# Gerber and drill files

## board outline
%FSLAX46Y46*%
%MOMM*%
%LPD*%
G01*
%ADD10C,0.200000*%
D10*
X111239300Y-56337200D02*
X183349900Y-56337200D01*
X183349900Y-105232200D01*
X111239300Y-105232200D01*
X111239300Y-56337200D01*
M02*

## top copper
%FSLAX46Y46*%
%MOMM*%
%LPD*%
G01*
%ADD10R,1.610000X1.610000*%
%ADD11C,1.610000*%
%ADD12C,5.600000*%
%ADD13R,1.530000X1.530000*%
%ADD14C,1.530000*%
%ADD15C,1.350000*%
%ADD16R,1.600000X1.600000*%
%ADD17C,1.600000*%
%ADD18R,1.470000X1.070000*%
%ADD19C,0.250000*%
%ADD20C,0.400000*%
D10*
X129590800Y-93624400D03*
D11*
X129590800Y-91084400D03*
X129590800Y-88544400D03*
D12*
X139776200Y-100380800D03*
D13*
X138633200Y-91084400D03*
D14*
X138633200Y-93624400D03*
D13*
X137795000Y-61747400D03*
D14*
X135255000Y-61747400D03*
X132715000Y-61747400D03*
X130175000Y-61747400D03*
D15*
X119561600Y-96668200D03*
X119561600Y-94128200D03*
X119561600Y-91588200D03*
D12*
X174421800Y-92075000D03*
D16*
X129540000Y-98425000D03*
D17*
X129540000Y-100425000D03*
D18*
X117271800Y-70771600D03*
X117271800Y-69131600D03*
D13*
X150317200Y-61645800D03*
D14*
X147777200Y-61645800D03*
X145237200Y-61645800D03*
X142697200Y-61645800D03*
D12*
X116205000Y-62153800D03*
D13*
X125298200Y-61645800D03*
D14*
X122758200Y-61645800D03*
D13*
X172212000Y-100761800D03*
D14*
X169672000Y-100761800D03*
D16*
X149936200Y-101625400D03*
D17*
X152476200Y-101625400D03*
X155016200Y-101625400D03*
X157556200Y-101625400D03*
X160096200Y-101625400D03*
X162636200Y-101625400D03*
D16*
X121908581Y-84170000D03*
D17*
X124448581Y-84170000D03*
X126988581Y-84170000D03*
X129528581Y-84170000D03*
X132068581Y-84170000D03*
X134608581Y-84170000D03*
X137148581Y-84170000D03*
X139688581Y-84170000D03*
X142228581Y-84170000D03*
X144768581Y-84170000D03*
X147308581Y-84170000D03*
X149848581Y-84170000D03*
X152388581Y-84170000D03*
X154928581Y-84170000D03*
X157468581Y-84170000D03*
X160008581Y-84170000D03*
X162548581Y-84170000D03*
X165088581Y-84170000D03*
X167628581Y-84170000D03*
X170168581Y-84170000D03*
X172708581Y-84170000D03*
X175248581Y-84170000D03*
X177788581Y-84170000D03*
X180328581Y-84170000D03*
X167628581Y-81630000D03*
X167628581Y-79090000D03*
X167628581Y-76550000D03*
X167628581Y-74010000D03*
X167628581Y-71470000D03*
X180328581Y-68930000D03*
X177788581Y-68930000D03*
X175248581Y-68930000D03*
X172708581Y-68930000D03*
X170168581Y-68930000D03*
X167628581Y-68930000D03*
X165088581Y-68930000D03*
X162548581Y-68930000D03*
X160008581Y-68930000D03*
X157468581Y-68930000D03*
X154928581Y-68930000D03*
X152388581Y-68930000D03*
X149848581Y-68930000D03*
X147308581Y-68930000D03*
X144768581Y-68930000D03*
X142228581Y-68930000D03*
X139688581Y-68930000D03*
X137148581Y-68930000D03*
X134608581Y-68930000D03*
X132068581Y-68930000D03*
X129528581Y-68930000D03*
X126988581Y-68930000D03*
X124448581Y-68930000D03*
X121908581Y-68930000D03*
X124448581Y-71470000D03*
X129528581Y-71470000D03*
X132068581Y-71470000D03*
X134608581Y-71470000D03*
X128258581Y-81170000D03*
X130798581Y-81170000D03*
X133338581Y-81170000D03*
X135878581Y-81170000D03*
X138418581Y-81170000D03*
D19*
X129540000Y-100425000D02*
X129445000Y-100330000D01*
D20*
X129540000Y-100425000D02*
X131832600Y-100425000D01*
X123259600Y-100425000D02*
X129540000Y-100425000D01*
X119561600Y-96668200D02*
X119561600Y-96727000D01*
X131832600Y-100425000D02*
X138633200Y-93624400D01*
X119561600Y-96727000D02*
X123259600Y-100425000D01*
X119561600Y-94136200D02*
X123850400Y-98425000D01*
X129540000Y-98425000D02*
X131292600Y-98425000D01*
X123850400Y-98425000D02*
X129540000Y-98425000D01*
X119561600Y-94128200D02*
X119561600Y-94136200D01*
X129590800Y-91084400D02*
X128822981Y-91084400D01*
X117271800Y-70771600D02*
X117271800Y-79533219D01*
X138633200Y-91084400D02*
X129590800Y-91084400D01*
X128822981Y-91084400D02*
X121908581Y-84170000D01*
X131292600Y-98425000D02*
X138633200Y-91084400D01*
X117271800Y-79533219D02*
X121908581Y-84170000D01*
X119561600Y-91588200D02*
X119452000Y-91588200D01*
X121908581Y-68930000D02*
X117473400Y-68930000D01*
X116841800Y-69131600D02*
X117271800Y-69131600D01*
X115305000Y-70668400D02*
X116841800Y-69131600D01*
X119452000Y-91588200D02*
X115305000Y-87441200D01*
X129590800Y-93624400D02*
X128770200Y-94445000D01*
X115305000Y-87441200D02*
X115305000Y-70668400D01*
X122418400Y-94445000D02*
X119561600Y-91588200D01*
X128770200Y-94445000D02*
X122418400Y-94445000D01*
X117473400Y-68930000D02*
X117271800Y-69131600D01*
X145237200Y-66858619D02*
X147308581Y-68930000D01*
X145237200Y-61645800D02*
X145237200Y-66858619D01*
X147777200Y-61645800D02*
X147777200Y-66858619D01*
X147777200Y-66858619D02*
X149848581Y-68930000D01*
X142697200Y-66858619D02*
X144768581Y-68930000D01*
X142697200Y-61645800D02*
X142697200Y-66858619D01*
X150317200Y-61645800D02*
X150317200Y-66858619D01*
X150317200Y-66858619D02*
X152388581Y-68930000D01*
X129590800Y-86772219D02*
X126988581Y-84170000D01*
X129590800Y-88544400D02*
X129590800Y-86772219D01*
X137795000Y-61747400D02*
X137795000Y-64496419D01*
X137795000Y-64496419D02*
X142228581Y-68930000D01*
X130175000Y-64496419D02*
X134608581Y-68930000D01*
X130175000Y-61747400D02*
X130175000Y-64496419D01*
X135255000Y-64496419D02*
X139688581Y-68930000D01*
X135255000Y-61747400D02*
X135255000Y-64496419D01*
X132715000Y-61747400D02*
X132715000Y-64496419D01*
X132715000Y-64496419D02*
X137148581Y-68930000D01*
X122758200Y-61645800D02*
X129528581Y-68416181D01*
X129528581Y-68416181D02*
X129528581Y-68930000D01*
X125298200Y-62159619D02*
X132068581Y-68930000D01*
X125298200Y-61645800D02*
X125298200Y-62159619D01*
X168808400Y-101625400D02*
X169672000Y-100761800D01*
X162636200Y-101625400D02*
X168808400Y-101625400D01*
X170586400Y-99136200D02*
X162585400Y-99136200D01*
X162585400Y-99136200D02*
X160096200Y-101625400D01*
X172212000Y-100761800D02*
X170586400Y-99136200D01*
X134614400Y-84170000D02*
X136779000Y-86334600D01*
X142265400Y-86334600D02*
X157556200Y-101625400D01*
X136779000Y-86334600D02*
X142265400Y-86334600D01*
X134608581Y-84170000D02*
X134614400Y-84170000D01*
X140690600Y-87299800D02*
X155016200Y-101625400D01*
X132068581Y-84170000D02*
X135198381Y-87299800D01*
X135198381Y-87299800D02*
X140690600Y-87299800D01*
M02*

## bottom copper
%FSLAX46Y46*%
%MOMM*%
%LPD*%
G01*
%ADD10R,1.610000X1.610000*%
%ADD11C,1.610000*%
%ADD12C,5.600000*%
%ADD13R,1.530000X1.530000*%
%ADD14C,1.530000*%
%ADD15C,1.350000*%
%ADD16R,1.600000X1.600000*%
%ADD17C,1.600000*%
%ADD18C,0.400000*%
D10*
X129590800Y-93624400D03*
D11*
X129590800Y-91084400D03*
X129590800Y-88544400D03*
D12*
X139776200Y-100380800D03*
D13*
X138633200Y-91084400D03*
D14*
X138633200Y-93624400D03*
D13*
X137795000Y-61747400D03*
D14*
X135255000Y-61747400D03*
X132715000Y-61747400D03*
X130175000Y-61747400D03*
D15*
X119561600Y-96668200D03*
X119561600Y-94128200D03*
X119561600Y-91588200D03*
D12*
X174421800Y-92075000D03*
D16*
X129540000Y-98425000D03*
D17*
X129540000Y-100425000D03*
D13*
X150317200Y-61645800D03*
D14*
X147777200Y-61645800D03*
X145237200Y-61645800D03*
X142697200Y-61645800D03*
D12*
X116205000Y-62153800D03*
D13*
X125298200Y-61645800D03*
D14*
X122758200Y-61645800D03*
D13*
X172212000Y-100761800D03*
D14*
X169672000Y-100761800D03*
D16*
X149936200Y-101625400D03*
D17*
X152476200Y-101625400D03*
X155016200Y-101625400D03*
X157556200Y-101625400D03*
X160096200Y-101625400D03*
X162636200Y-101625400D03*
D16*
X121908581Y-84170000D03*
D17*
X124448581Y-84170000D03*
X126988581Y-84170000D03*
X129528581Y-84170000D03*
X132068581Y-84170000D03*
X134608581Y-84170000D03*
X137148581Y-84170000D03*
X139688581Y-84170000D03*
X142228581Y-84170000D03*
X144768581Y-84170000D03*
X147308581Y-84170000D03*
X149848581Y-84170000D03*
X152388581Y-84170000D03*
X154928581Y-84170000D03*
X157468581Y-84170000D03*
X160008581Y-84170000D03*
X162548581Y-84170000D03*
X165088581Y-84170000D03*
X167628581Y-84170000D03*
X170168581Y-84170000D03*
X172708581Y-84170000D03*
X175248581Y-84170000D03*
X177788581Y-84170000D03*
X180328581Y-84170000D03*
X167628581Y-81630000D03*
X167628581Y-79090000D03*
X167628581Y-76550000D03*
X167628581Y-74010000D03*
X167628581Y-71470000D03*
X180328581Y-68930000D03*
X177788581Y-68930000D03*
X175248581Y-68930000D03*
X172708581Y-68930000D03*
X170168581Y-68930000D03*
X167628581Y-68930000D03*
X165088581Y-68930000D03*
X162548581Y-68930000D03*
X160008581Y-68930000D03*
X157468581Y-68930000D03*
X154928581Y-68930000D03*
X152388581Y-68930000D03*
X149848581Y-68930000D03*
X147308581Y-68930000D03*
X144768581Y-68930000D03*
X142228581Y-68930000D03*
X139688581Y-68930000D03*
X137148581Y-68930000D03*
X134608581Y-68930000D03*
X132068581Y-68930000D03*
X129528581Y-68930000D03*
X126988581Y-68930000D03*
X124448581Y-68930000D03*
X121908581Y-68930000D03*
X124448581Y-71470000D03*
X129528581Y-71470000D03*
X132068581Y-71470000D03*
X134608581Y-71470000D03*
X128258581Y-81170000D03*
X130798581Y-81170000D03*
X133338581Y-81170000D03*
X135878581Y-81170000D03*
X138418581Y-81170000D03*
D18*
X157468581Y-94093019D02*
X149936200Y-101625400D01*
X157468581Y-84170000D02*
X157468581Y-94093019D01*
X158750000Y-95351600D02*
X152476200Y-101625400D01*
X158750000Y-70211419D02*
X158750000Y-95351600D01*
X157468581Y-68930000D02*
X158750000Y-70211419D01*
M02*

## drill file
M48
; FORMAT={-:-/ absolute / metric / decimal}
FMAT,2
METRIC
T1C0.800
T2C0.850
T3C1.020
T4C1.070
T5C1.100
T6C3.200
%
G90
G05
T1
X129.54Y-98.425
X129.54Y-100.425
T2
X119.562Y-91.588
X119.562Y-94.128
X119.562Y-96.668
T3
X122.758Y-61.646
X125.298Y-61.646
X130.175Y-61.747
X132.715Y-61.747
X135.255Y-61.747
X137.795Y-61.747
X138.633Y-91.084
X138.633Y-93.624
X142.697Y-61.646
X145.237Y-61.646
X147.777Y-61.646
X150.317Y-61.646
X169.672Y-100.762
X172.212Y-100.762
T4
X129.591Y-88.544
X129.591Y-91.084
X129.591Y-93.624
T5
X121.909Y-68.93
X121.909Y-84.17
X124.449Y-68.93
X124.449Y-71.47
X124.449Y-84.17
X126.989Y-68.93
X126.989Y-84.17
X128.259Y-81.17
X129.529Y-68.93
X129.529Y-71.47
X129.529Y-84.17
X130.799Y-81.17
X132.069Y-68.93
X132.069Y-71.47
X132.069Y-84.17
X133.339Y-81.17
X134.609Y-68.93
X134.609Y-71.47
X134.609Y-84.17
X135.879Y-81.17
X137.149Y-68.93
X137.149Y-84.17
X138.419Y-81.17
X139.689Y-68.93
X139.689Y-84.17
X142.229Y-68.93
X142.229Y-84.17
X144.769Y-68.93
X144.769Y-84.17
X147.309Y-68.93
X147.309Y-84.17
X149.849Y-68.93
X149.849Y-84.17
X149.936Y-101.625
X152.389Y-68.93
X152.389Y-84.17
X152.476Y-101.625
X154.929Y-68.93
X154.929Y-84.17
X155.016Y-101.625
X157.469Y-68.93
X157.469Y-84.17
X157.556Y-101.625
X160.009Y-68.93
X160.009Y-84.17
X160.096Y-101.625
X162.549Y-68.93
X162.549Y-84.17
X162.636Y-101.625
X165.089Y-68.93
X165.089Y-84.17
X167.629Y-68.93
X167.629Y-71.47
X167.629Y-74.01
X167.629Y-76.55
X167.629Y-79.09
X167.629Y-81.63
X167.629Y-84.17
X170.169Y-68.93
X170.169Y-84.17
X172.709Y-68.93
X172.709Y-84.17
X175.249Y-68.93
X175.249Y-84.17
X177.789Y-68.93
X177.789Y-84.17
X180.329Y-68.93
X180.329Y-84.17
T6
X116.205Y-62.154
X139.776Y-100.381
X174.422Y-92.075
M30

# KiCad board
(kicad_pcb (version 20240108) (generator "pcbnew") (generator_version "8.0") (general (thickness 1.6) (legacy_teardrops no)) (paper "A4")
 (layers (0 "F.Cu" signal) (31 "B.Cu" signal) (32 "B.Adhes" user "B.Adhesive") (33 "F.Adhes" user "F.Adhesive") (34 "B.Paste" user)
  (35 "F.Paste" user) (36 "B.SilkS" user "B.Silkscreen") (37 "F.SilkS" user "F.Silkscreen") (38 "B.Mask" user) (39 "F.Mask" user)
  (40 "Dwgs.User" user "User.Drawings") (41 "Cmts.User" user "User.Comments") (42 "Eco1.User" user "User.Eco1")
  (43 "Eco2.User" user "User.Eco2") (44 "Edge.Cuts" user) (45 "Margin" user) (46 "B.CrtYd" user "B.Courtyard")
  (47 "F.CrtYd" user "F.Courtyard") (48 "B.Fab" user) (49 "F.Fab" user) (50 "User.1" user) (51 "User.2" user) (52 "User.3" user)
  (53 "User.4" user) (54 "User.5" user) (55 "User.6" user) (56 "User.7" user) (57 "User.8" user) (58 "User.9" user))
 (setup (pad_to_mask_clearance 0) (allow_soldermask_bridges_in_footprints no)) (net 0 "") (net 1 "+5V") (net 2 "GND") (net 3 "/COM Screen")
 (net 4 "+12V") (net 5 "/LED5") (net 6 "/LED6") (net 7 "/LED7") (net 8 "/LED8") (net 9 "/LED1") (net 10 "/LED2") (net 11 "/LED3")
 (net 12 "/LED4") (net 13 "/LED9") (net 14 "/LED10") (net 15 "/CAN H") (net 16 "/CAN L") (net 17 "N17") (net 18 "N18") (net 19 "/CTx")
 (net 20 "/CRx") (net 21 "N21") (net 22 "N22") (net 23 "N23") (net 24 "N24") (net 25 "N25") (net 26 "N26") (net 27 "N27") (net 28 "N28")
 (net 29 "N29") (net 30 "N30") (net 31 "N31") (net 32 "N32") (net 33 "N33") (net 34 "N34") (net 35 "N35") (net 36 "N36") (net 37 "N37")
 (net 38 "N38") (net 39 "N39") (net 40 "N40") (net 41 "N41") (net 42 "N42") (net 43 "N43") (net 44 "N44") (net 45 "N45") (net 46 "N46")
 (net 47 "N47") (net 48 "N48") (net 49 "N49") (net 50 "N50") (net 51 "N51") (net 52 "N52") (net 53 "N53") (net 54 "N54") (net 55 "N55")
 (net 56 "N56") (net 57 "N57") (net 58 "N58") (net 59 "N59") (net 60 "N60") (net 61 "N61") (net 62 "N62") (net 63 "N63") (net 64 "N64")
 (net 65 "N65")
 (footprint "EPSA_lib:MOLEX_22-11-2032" (layer "F.Cu") (at 129.5908 93.6244 90)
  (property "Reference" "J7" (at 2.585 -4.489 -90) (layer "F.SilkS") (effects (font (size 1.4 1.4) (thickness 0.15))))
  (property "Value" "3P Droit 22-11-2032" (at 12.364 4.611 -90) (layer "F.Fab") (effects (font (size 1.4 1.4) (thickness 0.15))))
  (pad "1" thru_hole rect (at 0 0 90) (size 1.61 1.61) (drill 1.07) (layers "*.Cu" "*.Mask") (remove_unused_layers no) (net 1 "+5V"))
  (pad "2" thru_hole circle (at 2.54 0 90) (size 1.61 1.61) (drill 1.07) (layers "*.Cu" "*.Mask") (remove_unused_layers no) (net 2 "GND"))
  (pad "3" thru_hole circle (at 5.08 0 90) (size 1.61 1.61) (drill 1.07) (layers "*.Cu" "*.Mask") (remove_unused_layers no)
   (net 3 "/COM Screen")))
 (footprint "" (layer "F.Cu") (at 139.7762 100.3808)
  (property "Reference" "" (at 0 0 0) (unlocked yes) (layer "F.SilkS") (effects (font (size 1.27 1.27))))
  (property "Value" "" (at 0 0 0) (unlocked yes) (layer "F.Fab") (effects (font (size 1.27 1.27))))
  (pad "1" thru_hole circle (at 0 0) (size 5.6 5.6) (drill 3.2) (layers "*.Cu" "*.Mask") (remove_unused_layers no)))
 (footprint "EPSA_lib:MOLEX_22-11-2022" (layer "F.Cu") (at 138.6332 91.0844 -90)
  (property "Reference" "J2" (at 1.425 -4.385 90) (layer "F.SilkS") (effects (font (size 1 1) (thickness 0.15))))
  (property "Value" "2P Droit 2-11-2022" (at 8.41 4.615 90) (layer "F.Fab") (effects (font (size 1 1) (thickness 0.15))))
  (pad "1" thru_hole rect (at 0 0 270) (size 1.53 1.53) (drill 1.02) (layers "*.Cu" "*.Mask") (remove_unused_layers no) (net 2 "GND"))
  (pad "2" thru_hole circle (at 2.54 0 270) (size 1.53 1.53) (drill 1.02) (layers "*.Cu" "*.Mask") (remove_unused_layers no) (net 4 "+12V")))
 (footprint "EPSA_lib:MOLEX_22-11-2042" (layer "F.Cu") (at 133.985 61.7474 180)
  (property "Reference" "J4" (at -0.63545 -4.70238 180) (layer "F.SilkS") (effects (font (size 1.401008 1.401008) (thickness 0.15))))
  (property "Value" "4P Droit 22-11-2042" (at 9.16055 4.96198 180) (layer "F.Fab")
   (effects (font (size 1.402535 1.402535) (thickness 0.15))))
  (pad "1" thru_hole rect (at -3.81 0 180) (size 1.53 1.53) (drill 1.02) (layers "*.Cu" "*.Mask") (remove_unused_layers no) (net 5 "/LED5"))
  (pad "2" thru_hole circle (at -1.27 0 180) (size 1.53 1.53) (drill 1.02) (layers "*.Cu" "*.Mask") (remove_unused_layers no)
   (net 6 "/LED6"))
  (pad "3" thru_hole circle (at 1.27 0 180) (size 1.53 1.53) (drill 1.02) (layers "*.Cu" "*.Mask") (remove_unused_layers no) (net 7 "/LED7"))
  (pad "4" thru_hole circle (at 3.81 0 180) (size 1.53 1.53) (drill 1.02) (layers "*.Cu" "*.Mask") (remove_unused_layers no) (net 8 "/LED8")))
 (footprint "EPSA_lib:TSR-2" (layer "F.Cu") (at 115.6716 101.1682 90)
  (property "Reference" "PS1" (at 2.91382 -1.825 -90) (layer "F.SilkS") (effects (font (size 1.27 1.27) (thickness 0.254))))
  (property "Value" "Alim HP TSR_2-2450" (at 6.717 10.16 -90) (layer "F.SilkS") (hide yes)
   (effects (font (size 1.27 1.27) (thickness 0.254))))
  (pad "1" thru_hole circle (at 4.5 3.89 90) (size 1.35 1.35) (drill 0.85) (layers "*.Cu" "*.Mask") (remove_unused_layers no) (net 4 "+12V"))
  (pad "2" thru_hole circle (at 7.04 3.89 90) (size 1.35 1.35) (drill 0.85) (layers "*.Cu" "*.Mask") (remove_unused_layers no) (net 2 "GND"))
  (pad "3" thru_hole circle (at 9.58 3.89 90) (size 1.35 1.35) (drill 0.85) (layers "*.Cu" "*.Mask") (remove_unused_layers no) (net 1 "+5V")))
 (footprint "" (layer "F.Cu") (at 174.4218 92.075)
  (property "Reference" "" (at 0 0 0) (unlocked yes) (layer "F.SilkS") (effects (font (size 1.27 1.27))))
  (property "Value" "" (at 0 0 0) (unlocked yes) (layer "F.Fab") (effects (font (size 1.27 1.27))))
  (pad "1" thru_hole circle (at 0 0) (size 5.6 5.6) (drill 3.2) (layers "*.Cu" "*.Mask") (remove_unused_layers no)))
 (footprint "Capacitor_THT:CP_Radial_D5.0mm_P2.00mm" (layer "F.Cu") (at 129.54 98.425 -90)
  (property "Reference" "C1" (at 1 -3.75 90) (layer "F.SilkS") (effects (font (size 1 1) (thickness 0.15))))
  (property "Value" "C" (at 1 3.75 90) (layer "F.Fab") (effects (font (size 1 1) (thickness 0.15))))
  (pad "1" thru_hole rect (at 0 0 270) (size 1.6 1.6) (drill 0.8) (layers "*.Cu" "*.Mask") (remove_unused_layers no) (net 2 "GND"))
  (pad "2" thru_hole circle (at 2 0 270) (size 1.6 1.6) (drill 0.8) (layers "*.Cu" "*.Mask") (remove_unused_layers no) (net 4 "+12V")))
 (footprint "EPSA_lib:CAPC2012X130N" (layer "F.Cu") (at 117.2718 69.9516 90)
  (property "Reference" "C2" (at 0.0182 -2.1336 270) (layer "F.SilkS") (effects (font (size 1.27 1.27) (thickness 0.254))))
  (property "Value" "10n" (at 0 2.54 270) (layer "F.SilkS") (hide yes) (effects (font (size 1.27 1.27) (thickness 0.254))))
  (pad "1" smd rect (at -0.82 0 90) (size 1.07 1.47) (layers "F.Cu" "F.Paste" "F.Mask") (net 2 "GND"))
  (pad "2" smd rect (at 0.82 0 90) (size 1.07 1.47) (layers "F.Cu" "F.Paste" "F.Mask") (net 1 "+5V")))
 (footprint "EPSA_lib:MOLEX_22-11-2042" (layer "F.Cu") (at 146.5072 61.6458 180)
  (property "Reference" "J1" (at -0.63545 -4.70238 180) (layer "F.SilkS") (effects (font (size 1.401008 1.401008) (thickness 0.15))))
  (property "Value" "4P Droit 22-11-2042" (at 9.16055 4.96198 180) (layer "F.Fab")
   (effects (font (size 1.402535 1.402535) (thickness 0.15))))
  (pad "1" thru_hole rect (at -3.81 0 180) (size 1.53 1.53) (drill 1.02) (layers "*.Cu" "*.Mask") (remove_unused_layers no) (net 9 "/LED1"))
  (pad "2" thru_hole circle (at -1.27 0 180) (size 1.53 1.53) (drill 1.02) (layers "*.Cu" "*.Mask") (remove_unused_layers no)
   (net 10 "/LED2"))
  (pad "3" thru_hole circle (at 1.27 0 180) (size 1.53 1.53) (drill 1.02) (layers "*.Cu" "*.Mask") (remove_unused_layers no)
   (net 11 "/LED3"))
  (pad "4" thru_hole circle (at 3.81 0 180) (size 1.53 1.53) (drill 1.02) (layers "*.Cu" "*.Mask") (remove_unused_layers no)
   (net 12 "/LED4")))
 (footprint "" (layer "F.Cu") (at 116.205 62.1538)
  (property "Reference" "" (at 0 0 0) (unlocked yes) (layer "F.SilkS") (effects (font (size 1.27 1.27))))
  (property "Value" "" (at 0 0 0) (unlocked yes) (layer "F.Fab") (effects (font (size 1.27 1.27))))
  (pad "1" thru_hole circle (at 0 0) (size 5.6 5.6) (drill 3.2) (layers "*.Cu" "*.Mask") (remove_unused_layers no)))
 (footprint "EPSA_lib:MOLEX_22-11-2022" (layer "F.Cu") (at 125.2982 61.6458 180)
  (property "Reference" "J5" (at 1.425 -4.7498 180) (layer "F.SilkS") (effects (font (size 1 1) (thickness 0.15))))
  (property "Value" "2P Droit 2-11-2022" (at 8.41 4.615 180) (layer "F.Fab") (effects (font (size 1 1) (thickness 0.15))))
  (pad "1" thru_hole rect (at 0 0 180) (size 1.53 1.53) (drill 1.02) (layers "*.Cu" "*.Mask") (remove_unused_layers no) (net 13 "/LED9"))
  (pad "2" thru_hole circle (at 2.54 0 180) (size 1.53 1.53) (drill 1.02) (layers "*.Cu" "*.Mask") (remove_unused_layers no)
   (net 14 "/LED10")))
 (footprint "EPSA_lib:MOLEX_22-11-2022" (layer "F.Cu") (at 172.212 100.7618 180)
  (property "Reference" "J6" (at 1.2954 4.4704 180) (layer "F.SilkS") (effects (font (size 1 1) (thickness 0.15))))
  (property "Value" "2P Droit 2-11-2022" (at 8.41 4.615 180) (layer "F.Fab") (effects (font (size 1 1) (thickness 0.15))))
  (pad "1" thru_hole rect (at 0 0 180) (size 1.53 1.53) (drill 1.02) (layers "*.Cu" "*.Mask") (remove_unused_layers no) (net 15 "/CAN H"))
  (pad "2" thru_hole circle (at 2.54 0 180) (size 1.53 1.53) (drill 1.02) (layers "*.Cu" "*.Mask") (remove_unused_layers no)
   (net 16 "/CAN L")))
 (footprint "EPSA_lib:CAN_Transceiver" (layer "F.Cu") (at 147.3962 104.1654)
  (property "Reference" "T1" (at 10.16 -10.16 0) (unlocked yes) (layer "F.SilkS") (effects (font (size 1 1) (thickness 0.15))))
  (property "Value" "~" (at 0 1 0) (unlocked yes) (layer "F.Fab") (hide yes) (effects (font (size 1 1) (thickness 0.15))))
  (pad "1" thru_hole rect (at 2.54 -2.54) (size 1.6 1.6) (drill 1.1) (layers "*.Cu" "*.Mask") (remove_unused_layers no) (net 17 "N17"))
  (pad "2" thru_hole circle (at 5.08 -2.54) (size 1.6 1.6) (drill 1.1) (layers "*.Cu" "*.Mask") (remove_unused_layers no) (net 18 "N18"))
  (pad "3" thru_hole circle (at 7.62 -2.54) (size 1.6 1.6) (drill 1.1) (layers "*.Cu" "*.Mask") (remove_unused_layers no) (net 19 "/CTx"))
  (pad "4" thru_hole circle (at 10.16 -2.54) (size 1.6 1.6) (drill 1.1) (layers "*.Cu" "*.Mask") (remove_unused_layers no) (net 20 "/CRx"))
  (pad "5" thru_hole circle (at 12.7 -2.54) (size 1.6 1.6) (drill 1.1) (layers "*.Cu" "*.Mask") (remove_unused_layers no) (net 15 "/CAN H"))
  (pad "6" thru_hole circle (at 15.24 -2.54) (size 1.6 1.6) (drill 1.1) (layers "*.Cu" "*.Mask") (remove_unused_layers no) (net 16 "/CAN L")))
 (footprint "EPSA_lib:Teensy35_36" (layer "F.Cu") (at 151.118581 76.55)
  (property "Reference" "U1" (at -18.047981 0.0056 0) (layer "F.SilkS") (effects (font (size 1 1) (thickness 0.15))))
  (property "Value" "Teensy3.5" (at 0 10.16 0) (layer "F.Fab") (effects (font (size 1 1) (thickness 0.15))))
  (pad "1" thru_hole rect (at -29.21 7.62) (size 1.6 1.6) (drill 1.1) (layers "*.Cu" "*.Mask") (remove_unused_layers no) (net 2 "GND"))
  (pad "2" thru_hole circle (at -26.67 7.62) (size 1.6 1.6) (drill 1.1) (layers "*.Cu" "*.Mask") (remove_unused_layers no) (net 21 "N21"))
  (pad "3" thru_hole circle (at -24.13 7.62) (size 1.6 1.6) (drill 1.1) (layers "*.Cu" "*.Mask") (remove_unused_layers no)
   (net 3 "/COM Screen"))
  (pad "4" thru_hole circle (at -21.59 7.62) (size 1.6 1.6) (drill 1.1) (layers "*.Cu" "*.Mask") (remove_unused_layers no) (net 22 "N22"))
  (pad "5" thru_hole circle (at -19.05 7.62) (size 1.6 1.6) (drill 1.1) (layers "*.Cu" "*.Mask") (remove_unused_layers no) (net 19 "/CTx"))
  (pad "6" thru_hole circle (at -16.51 7.62) (size 1.6 1.6) (drill 1.1) (layers "*.Cu" "*.Mask") (remove_unused_layers no) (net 20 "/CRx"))
  (pad "7" thru_hole circle (at -13.97 7.62) (size 1.6 1.6) (drill 1.1) (layers "*.Cu" "*.Mask") (remove_unused_layers no) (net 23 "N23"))
  (pad "8" thru_hole circle (at -11.43 7.62) (size 1.6 1.6) (drill 1.1) (layers "*.Cu" "*.Mask") (remove_unused_layers no) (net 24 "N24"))
  (pad "9" thru_hole circle (at -8.89 7.62) (size 1.6 1.6) (drill 1.1) (layers "*.Cu" "*.Mask") (remove_unused_layers no) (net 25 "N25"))
  (pad "10" thru_hole circle (at -6.35 7.62) (size 1.6 1.6) (drill 1.1) (layers "*.Cu" "*.Mask") (remove_unused_layers no) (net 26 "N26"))
  (pad "11" thru_hole circle (at -3.81 7.62) (size 1.6 1.6) (drill 1.1) (layers "*.Cu" "*.Mask") (remove_unused_layers no) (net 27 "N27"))
  (pad "12" thru_hole circle (at -1.27 7.62) (size 1.6 1.6) (drill 1.1) (layers "*.Cu" "*.Mask") (remove_unused_layers no) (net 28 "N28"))
  (pad "13" thru_hole circle (at 1.27 7.62) (size 1.6 1.6) (drill 1.1) (layers "*.Cu" "*.Mask") (remove_unused_layers no) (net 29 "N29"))
  (pad "14" thru_hole circle (at 3.81 7.62) (size 1.6 1.6) (drill 1.1) (layers "*.Cu" "*.Mask") (remove_unused_layers no) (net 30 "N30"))
  (pad "15" thru_hole circle (at 6.35 7.62) (size 1.6 1.6) (drill 1.1) (layers "*.Cu" "*.Mask") (remove_unused_layers no) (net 17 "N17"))
  (pad "16" thru_hole circle (at 8.89 7.62) (size 1.6 1.6) (drill 1.1) (layers "*.Cu" "*.Mask") (remove_unused_layers no) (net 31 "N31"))
  (pad "17" thru_hole circle (at 11.43 7.62) (size 1.6 1.6) (drill 1.1) (layers "*.Cu" "*.Mask") (remove_unused_layers no) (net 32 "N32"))
  (pad "18" thru_hole circle (at 13.97 7.62) (size 1.6 1.6) (drill 1.1) (layers "*.Cu" "*.Mask") (remove_unused_layers no) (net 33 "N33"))
  (pad "19" thru_hole circle (at 16.51 7.62) (size 1.6 1.6) (drill 1.1) (layers "*.Cu" "*.Mask") (remove_unused_layers no) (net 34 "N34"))
  (pad "20" thru_hole circle (at 19.05 7.62) (size 1.6 1.6) (drill 1.1) (layers "*.Cu" "*.Mask") (remove_unused_layers no) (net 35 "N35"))
  (pad "21" thru_hole circle (at 21.59 7.62) (size 1.6 1.6) (drill 1.1) (layers "*.Cu" "*.Mask") (remove_unused_layers no) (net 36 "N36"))
  (pad "22" thru_hole circle (at 24.13 7.62) (size 1.6 1.6) (drill 1.1) (layers "*.Cu" "*.Mask") (remove_unused_layers no) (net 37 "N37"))
  (pad "23" thru_hole circle (at 26.67 7.62) (size 1.6 1.6) (drill 1.1) (layers "*.Cu" "*.Mask") (remove_unused_layers no) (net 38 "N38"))
  (pad "24" thru_hole circle (at 29.21 7.62) (size 1.6 1.6) (drill 1.1) (layers "*.Cu" "*.Mask") (remove_unused_layers no) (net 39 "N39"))
  (pad "25" thru_hole circle (at 16.51 5.08) (size 1.6 1.6) (drill 1.1) (layers "*.Cu" "*.Mask") (remove_unused_layers no) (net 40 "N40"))
  (pad "26" thru_hole circle (at 16.51 2.54) (size 1.6 1.6) (drill 1.1) (layers "*.Cu" "*.Mask") (remove_unused_layers no) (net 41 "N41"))
  (pad "27" thru_hole circle (at 16.51 0) (size 1.6 1.6) (drill 1.1) (layers "*.Cu" "*.Mask") (remove_unused_layers no) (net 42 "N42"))
  (pad "28" thru_hole circle (at 16.51 -2.54) (size 1.6 1.6) (drill 1.1) (layers "*.Cu" "*.Mask") (remove_unused_layers no) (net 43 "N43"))
  (pad "29" thru_hole circle (at 16.51 -5.08) (size 1.6 1.6) (drill 1.1) (layers "*.Cu" "*.Mask") (remove_unused_layers no) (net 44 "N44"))
  (pad "30" thru_hole circle (at 29.21 -7.62) (size 1.6 1.6) (drill 1.1) (layers "*.Cu" "*.Mask") (remove_unused_layers no) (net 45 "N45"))
  (pad "31" thru_hole circle (at 26.67 -7.62) (size 1.6 1.6) (drill 1.1) (layers "*.Cu" "*.Mask") (remove_unused_layers no) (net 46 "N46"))
  (pad "32" thru_hole circle (at 24.13 -7.62) (size 1.6 1.6) (drill 1.1) (layers "*.Cu" "*.Mask") (remove_unused_layers no) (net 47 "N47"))
  (pad "33" thru_hole circle (at 21.59 -7.62) (size 1.6 1.6) (drill 1.1) (layers "*.Cu" "*.Mask") (remove_unused_layers no) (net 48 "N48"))
  (pad "34" thru_hole circle (at 19.05 -7.62) (size 1.6 1.6) (drill 1.1) (layers "*.Cu" "*.Mask") (remove_unused_layers no) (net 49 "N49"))
  (pad "35" thru_hole circle (at 16.51 -7.62) (size 1.6 1.6) (drill 1.1) (layers "*.Cu" "*.Mask") (remove_unused_layers no) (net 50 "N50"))
  (pad "36" thru_hole circle (at 13.97 -7.62) (size 1.6 1.6) (drill 1.1) (layers "*.Cu" "*.Mask") (remove_unused_layers no) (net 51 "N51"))
  (pad "37" thru_hole circle (at 11.43 -7.62) (size 1.6 1.6) (drill 1.1) (layers "*.Cu" "*.Mask") (remove_unused_layers no) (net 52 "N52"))
  (pad "38" thru_hole circle (at 8.89 -7.62) (size 1.6 1.6) (drill 1.1) (layers "*.Cu" "*.Mask") (remove_unused_layers no) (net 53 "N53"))
  (pad "39" thru_hole circle (at 6.35 -7.62) (size 1.6 1.6) (drill 1.1) (layers "*.Cu" "*.Mask") (remove_unused_layers no) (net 18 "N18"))
  (pad "40" thru_hole circle (at 3.81 -7.62) (size 1.6 1.6) (drill 1.1) (layers "*.Cu" "*.Mask") (remove_unused_layers no) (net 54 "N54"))
  (pad "41" thru_hole circle (at 1.27 -7.62) (size 1.6 1.6) (drill 1.1) (layers "*.Cu" "*.Mask") (remove_unused_layers no) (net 9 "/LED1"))
  (pad "42" thru_hole circle (at -1.27 -7.62) (size 1.6 1.6) (drill 1.1) (layers "*.Cu" "*.Mask") (remove_unused_layers no) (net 10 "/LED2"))
  (pad "43" thru_hole circle (at -3.81 -7.62) (size 1.6 1.6) (drill 1.1) (layers "*.Cu" "*.Mask") (remove_unused_layers no) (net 11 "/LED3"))
  (pad "44" thru_hole circle (at -6.35 -7.62) (size 1.6 1.6) (drill 1.1) (layers "*.Cu" "*.Mask") (remove_unused_layers no) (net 12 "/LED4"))
  (pad "45" thru_hole circle (at -8.89 -7.62) (size 1.6 1.6) (drill 1.1) (layers "*.Cu" "*.Mask") (remove_unused_layers no) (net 5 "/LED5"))
  (pad "46" thru_hole circle (at -11.43 -7.62) (size 1.6 1.6) (drill 1.1) (layers "*.Cu" "*.Mask") (remove_unused_layers no) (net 6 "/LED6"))
  (pad "47" thru_hole circle (at -13.97 -7.62) (size 1.6 1.6) (drill 1.1) (layers "*.Cu" "*.Mask") (remove_unused_layers no) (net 7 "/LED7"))
  (pad "48" thru_hole circle (at -16.51 -7.62) (size 1.6 1.6) (drill 1.1) (layers "*.Cu" "*.Mask") (remove_unused_layers no) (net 8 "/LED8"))
  (pad "49" thru_hole circle (at -19.05 -7.62) (size 1.6 1.6) (drill 1.1) (layers "*.Cu" "*.Mask") (remove_unused_layers no)
   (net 13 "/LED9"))
  (pad "50" thru_hole circle (at -21.59 -7.62) (size 1.6 1.6) (drill 1.1) (layers "*.Cu" "*.Mask") (remove_unused_layers no)
   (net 14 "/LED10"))
  (pad "51" thru_hole circle (at -24.13 -7.62) (size 1.6 1.6) (drill 1.1) (layers "*.Cu" "*.Mask") (remove_unused_layers no) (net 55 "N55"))
  (pad "52" thru_hole circle (at -26.67 -7.62) (size 1.6 1.6) (drill 1.1) (layers "*.Cu" "*.Mask") (remove_unused_layers no) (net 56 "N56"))
  (pad "53" thru_hole circle (at -29.21 -7.62) (size 1.6 1.6) (drill 1.1) (layers "*.Cu" "*.Mask") (remove_unused_layers no) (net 1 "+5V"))
  (pad "54" thru_hole circle (at -26.67 -5.08) (size 1.6 1.6) (drill 1.1) (layers "*.Cu" "*.Mask") (remove_unused_layers no) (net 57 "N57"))
  (pad "55" thru_hole circle (at -21.59 -5.08) (size 1.6 1.6) (drill 1.1) (layers "*.Cu" "*.Mask") (remove_unused_layers no) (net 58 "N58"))
  (pad "56" thru_hole circle (at -19.05 -5.08) (size 1.6 1.6) (drill 1.1) (layers "*.Cu" "*.Mask") (remove_unused_layers no) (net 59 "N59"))
  (pad "57" thru_hole circle (at -16.51 -5.08) (size 1.6 1.6) (drill 1.1) (layers "*.Cu" "*.Mask") (remove_unused_layers no) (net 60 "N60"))
  (pad "58" thru_hole circle (at -22.86 4.62) (size 1.6 1.6) (drill 1.1) (layers "*.Cu" "*.Mask") (remove_unused_layers no) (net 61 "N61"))
  (pad "59" thru_hole circle (at -20.32 4.62) (size 1.6 1.6) (drill 1.1) (layers "*.Cu" "*.Mask") (remove_unused_layers no) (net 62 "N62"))
  (pad "60" thru_hole circle (at -17.78 4.62) (size 1.6 1.6) (drill 1.1) (layers "*.Cu" "*.Mask") (remove_unused_layers no) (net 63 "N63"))
  (pad "61" thru_hole circle (at -15.24 4.62) (size 1.6 1.6) (drill 1.1) (layers "*.Cu" "*.Mask") (remove_unused_layers no) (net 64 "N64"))
  (pad "62" thru_hole circle (at -12.7 4.62) (size 1.6 1.6) (drill 1.1) (layers "*.Cu" "*.Mask") (remove_unused_layers no) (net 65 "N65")))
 (gr_rect (start 111.2393 56.3372) (end 183.3499 105.2322) (stroke (width 0.2) (type default)) (fill none) (layer "Edge.Cuts"))
 (segment (start 129.54 100.425) (end 129.445 100.33) (width 0.25) (layer "F.Cu") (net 4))
 (segment (start 129.54 100.425) (end 131.8326 100.425) (width 0.4) (layer "F.Cu") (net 4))
 (segment (start 123.2596 100.425) (end 129.54 100.425) (width 0.4) (layer "F.Cu") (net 4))
 (segment (start 119.5616 96.6682) (end 119.5616 96.727) (width 0.4) (layer "F.Cu") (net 4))
 (segment (start 131.8326 100.425) (end 138.6332 93.6244) (width 0.4) (layer "F.Cu") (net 4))
 (segment (start 119.5616 96.727) (end 123.2596 100.425) (width 0.4) (layer "F.Cu") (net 4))
 (segment (start 119.5616 94.1362) (end 123.8504 98.425) (width 0.4) (layer "F.Cu") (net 2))
 (segment (start 129.54 98.425) (end 131.2926 98.425) (width 0.4) (layer "F.Cu") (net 2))
 (segment (start 123.8504 98.425) (end 129.54 98.425) (width 0.4) (layer "F.Cu") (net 2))
 (segment (start 119.5616 94.1282) (end 119.5616 94.1362) (width 0.4) (layer "F.Cu") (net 2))
 (segment (start 129.5908 91.0844) (end 128.822981 91.0844) (width 0.4) (layer "F.Cu") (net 2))
 (segment (start 117.2718 70.7716) (end 117.2718 79.533219) (width 0.4) (layer "F.Cu") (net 2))
 (segment (start 138.6332 91.0844) (end 129.5908 91.0844) (width 0.4) (layer "F.Cu") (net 2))
 (segment (start 128.822981 91.0844) (end 121.908581 84.17) (width 0.4) (layer "F.Cu") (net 2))
 (segment (start 131.2926 98.425) (end 138.6332 91.0844) (width 0.4) (layer "F.Cu") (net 2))
 (segment (start 117.2718 79.533219) (end 121.908581 84.17) (width 0.4) (layer "F.Cu") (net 2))
 (segment (start 119.5616 91.5882) (end 119.452 91.5882) (width 0.4) (layer "F.Cu") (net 1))
 (segment (start 121.908581 68.93) (end 117.4734 68.93) (width 0.4) (layer "F.Cu") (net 1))
 (segment (start 116.8418 69.1316) (end 117.2718 69.1316) (width 0.4) (layer "F.Cu") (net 1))
 (segment (start 115.305 70.6684) (end 116.8418 69.1316) (width 0.4) (layer "F.Cu") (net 1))
 (segment (start 119.452 91.5882) (end 115.305 87.4412) (width 0.4) (layer "F.Cu") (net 1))
 (segment (start 129.5908 93.6244) (end 128.7702 94.445) (width 0.4) (layer "F.Cu") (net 1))
 (segment (start 115.305 87.4412) (end 115.305 70.6684) (width 0.4) (layer "F.Cu") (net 1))
 (segment (start 122.4184 94.445) (end 119.5616 91.5882) (width 0.4) (layer "F.Cu") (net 1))
 (segment (start 128.7702 94.445) (end 122.4184 94.445) (width 0.4) (layer "F.Cu") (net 1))
 (segment (start 117.4734 68.93) (end 117.2718 69.1316) (width 0.4) (layer "F.Cu") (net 1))
 (segment (start 145.2372 66.858619) (end 147.308581 68.93) (width 0.4) (layer "F.Cu") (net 11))
 (segment (start 145.2372 61.6458) (end 145.2372 66.858619) (width 0.4) (layer "F.Cu") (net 11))
 (segment (start 147.7772 61.6458) (end 147.7772 66.858619) (width 0.4) (layer "F.Cu") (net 10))
 (segment (start 147.7772 66.858619) (end 149.848581 68.93) (width 0.4) (layer "F.Cu") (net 10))
 (segment (start 142.6972 66.858619) (end 144.768581 68.93) (width 0.4) (layer "F.Cu") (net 12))
 (segment (start 142.6972 61.6458) (end 142.6972 66.858619) (width 0.4) (layer "F.Cu") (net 12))
 (segment (start 150.3172 61.6458) (end 150.3172 66.858619) (width 0.4) (layer "F.Cu") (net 9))
 (segment (start 150.3172 66.858619) (end 152.388581 68.93) (width 0.4) (layer "F.Cu") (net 9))
 (segment (start 129.5908 86.772219) (end 126.988581 84.17) (width 0.4) (layer "F.Cu") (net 3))
 (segment (start 129.5908 88.5444) (end 129.5908 86.772219) (width 0.4) (layer "F.Cu") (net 3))
 (segment (start 137.795 61.7474) (end 137.795 64.496419) (width 0.4) (layer "F.Cu") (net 5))
 (segment (start 137.795 64.496419) (end 142.228581 68.93) (width 0.4) (layer "F.Cu") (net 5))
 (segment (start 130.175 64.496419) (end 134.608581 68.93) (width 0.4) (layer "F.Cu") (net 8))
 (segment (start 130.175 61.7474) (end 130.175 64.496419) (width 0.4) (layer "F.Cu") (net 8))
 (segment (start 135.255 64.496419) (end 139.688581 68.93) (width 0.4) (layer "F.Cu") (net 6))
 (segment (start 135.255 61.7474) (end 135.255 64.496419) (width 0.4) (layer "F.Cu") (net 6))
 (segment (start 132.715 61.7474) (end 132.715 64.496419) (width 0.4) (layer "F.Cu") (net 7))
 (segment (start 132.715 64.496419) (end 137.148581 68.93) (width 0.4) (layer "F.Cu") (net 7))
 (segment (start 122.7582 61.6458) (end 129.528581 68.416181) (width 0.4) (layer "F.Cu") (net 14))
 (segment (start 129.528581 68.416181) (end 129.528581 68.93) (width 0.4) (layer "F.Cu") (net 14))
 (segment (start 125.2982 62.159619) (end 132.068581 68.93) (width 0.4) (layer "F.Cu") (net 13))
 (segment (start 125.2982 61.6458) (end 125.2982 62.159619) (width 0.4) (layer "F.Cu") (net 13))
 (segment (start 168.8084 101.6254) (end 169.672 100.7618) (width 0.4) (layer "F.Cu") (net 16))
 (segment (start 162.6362 101.6254) (end 168.8084 101.6254) (width 0.4) (layer "F.Cu") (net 16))
 (segment (start 170.5864 99.1362) (end 162.5854 99.1362) (width 0.4) (layer "F.Cu") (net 15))
 (segment (start 162.5854 99.1362) (end 160.0962 101.6254) (width 0.4) (layer "F.Cu") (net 15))
 (segment (start 172.212 100.7618) (end 170.5864 99.1362) (width 0.4) (layer "F.Cu") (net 15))
 (segment (start 134.6144 84.17) (end 136.779 86.3346) (width 0.4) (layer "F.Cu") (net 20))
 (segment (start 142.2654 86.3346) (end 157.5562 101.6254) (width 0.4) (layer "F.Cu") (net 20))
 (segment (start 136.779 86.3346) (end 142.2654 86.3346) (width 0.4) (layer "F.Cu") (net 20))
 (segment (start 134.608581 84.17) (end 134.6144 84.17) (width 0.4) (layer "F.Cu") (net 20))
 (segment (start 157.468581 94.093019) (end 149.9362 101.6254) (width 0.4) (layer "B.Cu") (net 17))
 (segment (start 157.468581 84.17) (end 157.468581 94.093019) (width 0.4) (layer "B.Cu") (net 17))
 (segment (start 140.6906 87.2998) (end 155.0162 101.6254) (width 0.4) (layer "F.Cu") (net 19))
 (segment (start 132.068581 84.17) (end 135.198381 87.2998) (width 0.4) (layer "F.Cu") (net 19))
 (segment (start 135.198381 87.2998) (end 140.6906 87.2998) (width 0.4) (layer "F.Cu") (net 19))
 (segment (start 158.75 95.3516) (end 152.4762 101.6254) (width 0.4) (layer "B.Cu") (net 18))
 (segment (start 158.75 70.211419) (end 158.75 95.3516) (width 0.4) (layer "B.Cu") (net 18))
 (segment (start 157.468581 68.93) (end 158.75 70.211419) (width 0.4) (layer "B.Cu") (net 18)))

